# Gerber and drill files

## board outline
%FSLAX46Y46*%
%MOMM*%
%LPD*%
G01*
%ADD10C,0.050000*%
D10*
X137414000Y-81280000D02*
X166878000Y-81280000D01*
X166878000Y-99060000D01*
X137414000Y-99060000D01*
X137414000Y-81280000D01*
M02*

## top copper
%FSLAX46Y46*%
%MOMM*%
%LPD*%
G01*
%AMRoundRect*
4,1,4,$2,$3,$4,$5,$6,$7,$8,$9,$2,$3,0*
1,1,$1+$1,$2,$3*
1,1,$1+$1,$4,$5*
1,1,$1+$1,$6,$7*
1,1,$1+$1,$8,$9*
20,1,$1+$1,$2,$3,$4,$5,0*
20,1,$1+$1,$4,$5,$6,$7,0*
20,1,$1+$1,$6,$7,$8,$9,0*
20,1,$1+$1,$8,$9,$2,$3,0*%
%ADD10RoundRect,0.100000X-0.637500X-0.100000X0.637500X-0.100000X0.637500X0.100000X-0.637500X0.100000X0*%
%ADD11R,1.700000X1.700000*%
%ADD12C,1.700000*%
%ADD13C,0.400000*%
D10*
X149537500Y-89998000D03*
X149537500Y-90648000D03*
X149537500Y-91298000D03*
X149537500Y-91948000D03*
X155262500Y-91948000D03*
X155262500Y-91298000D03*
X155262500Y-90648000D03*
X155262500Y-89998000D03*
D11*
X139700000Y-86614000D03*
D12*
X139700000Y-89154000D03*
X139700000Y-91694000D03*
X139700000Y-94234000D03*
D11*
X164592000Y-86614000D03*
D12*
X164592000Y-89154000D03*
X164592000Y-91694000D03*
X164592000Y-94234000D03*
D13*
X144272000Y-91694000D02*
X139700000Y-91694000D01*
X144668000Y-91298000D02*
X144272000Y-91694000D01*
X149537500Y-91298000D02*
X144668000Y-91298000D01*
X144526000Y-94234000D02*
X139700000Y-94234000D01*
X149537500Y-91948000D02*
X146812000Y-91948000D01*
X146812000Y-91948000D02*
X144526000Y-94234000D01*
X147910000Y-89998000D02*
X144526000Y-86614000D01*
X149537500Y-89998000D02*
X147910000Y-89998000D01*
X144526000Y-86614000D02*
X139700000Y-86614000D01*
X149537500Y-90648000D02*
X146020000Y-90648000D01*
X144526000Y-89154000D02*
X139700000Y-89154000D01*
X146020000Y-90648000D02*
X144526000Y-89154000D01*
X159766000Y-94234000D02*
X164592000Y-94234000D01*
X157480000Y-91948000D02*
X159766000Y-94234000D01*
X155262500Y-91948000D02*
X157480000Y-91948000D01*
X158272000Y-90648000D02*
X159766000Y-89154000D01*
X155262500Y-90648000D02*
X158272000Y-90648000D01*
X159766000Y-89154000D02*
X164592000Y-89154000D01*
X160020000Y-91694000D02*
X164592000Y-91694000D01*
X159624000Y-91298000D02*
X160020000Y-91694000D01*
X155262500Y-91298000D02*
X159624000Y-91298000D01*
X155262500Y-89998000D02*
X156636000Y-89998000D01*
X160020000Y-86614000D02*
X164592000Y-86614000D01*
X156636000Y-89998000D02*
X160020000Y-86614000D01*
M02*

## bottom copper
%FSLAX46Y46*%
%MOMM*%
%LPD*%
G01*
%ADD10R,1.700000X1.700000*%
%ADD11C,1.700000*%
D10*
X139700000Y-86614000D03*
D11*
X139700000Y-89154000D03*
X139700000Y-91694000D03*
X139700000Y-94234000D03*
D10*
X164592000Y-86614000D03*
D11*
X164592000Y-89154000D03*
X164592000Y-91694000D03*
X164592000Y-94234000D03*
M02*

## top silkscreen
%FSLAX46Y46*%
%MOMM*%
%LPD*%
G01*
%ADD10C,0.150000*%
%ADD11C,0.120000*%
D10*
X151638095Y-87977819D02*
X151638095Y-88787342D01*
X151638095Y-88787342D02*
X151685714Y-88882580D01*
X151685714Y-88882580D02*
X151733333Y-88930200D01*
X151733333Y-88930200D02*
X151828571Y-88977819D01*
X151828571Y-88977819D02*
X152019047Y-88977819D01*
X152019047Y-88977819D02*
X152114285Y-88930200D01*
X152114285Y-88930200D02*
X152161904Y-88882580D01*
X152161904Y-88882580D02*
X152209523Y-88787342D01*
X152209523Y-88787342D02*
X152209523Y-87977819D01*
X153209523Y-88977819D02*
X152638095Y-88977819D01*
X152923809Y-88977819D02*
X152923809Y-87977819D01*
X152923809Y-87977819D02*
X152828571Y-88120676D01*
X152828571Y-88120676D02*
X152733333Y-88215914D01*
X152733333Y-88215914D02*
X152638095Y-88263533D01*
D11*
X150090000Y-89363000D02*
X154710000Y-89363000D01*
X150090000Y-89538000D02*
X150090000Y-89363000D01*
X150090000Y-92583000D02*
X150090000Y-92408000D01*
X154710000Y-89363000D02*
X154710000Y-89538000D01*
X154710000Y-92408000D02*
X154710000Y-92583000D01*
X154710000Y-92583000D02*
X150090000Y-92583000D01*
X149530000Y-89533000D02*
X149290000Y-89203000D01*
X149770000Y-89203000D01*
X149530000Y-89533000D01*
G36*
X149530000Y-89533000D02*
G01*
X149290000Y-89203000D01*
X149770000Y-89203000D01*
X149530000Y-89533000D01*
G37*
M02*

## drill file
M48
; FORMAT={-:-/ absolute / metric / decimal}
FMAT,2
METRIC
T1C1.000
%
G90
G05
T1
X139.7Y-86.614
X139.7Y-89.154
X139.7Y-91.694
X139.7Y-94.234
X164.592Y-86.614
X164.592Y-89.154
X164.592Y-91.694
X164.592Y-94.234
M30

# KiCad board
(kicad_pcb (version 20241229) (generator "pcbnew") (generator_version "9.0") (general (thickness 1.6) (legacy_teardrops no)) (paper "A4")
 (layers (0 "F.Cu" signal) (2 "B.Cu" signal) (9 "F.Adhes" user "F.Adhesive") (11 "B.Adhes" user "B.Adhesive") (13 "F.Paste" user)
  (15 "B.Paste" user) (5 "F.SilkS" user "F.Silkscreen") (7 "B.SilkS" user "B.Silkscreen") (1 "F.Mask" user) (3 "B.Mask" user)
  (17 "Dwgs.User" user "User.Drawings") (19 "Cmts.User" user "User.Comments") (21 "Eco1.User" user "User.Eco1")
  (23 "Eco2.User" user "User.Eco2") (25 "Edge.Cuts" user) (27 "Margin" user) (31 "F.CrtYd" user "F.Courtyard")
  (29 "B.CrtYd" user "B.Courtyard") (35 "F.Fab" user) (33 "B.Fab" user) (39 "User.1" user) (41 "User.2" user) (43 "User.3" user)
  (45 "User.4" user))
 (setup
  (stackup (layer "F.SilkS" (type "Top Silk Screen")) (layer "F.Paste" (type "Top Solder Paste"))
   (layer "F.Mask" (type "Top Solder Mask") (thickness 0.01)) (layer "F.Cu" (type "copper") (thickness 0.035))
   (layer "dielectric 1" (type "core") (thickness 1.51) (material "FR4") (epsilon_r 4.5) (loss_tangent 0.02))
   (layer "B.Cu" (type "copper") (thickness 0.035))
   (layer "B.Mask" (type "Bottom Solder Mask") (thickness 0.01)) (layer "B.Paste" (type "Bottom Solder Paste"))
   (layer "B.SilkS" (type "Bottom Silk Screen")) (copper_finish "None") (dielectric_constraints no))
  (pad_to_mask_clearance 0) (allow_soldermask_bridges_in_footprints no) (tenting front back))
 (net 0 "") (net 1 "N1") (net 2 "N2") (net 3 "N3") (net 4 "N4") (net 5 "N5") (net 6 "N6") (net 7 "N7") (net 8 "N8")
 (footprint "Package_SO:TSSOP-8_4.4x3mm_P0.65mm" (layer "F.Cu") (at 152.4 90.973)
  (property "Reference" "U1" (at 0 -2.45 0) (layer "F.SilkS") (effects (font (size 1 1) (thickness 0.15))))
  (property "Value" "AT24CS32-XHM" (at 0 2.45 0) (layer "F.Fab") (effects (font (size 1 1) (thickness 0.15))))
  (fp_line (start -2.31 -1.61) (end 2.31 -1.61) (stroke (width 0.12) (type solid)) (layer "F.SilkS"))
  (fp_line (start -2.31 -1.435) (end -2.31 -1.61) (stroke (width 0.12) (type solid)) (layer "F.SilkS"))
  (fp_line (start -2.31 1.61) (end -2.31 1.435) (stroke (width 0.12) (type solid)) (layer "F.SilkS"))
  (fp_line (start 2.31 -1.61) (end 2.31 -1.435) (stroke (width 0.12) (type solid)) (layer "F.SilkS"))
  (fp_line (start 2.31 1.435) (end 2.31 1.61) (stroke (width 0.12) (type solid)) (layer "F.SilkS"))
  (fp_line (start 2.31 1.61) (end -2.31 1.61) (stroke (width 0.12) (type solid)) (layer "F.SilkS"))
  (fp_poly (pts (xy -2.87 -1.44) (xy -3.11 -1.77) (xy -2.63 -1.77)) (stroke (width 0.12) (type solid)) (fill yes) (layer "F.SilkS"))
  (pad "1" smd roundrect (at -2.8625 -0.975) (size 1.475 0.4) (layers "F.Cu" "F.Mask" "F.Paste") (roundrect_rratio 0.25) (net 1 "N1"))
  (pad "2" smd roundrect (at -2.8625 -0.325) (size 1.475 0.4) (layers "F.Cu" "F.Mask" "F.Paste") (roundrect_rratio 0.25) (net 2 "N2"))
  (pad "3" smd roundrect (at -2.8625 0.325) (size 1.475 0.4) (layers "F.Cu" "F.Mask" "F.Paste") (roundrect_rratio 0.25) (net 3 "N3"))
  (pad "4" smd roundrect (at -2.8625 0.975) (size 1.475 0.4) (layers "F.Cu" "F.Mask" "F.Paste") (roundrect_rratio 0.25) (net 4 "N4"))
  (pad "5" smd roundrect (at 2.8625 0.975) (size 1.475 0.4) (layers "F.Cu" "F.Mask" "F.Paste") (roundrect_rratio 0.25) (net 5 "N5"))
  (pad "6" smd roundrect (at 2.8625 0.325) (size 1.475 0.4) (layers "F.Cu" "F.Mask" "F.Paste") (roundrect_rratio 0.25) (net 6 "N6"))
  (pad "7" smd roundrect (at 2.8625 -0.325) (size 1.475 0.4) (layers "F.Cu" "F.Mask" "F.Paste") (roundrect_rratio 0.25) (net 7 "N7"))
  (pad "8" smd roundrect (at 2.8625 -0.975) (size 1.475 0.4) (layers "F.Cu" "F.Mask" "F.Paste") (roundrect_rratio 0.25) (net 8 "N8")))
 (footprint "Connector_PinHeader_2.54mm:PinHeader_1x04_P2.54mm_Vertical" (layer "B.Cu") (at 139.7 86.614 180)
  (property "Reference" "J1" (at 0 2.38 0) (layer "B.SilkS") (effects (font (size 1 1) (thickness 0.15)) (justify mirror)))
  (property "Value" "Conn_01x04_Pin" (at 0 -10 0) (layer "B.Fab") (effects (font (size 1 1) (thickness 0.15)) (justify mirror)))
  (pad "1" thru_hole rect (at 0 0 180) (size 1.7 1.7) (drill 1) (layers "*.Cu" "*.Mask") (remove_unused_layers no) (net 1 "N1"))
  (pad "2" thru_hole circle (at 0 -2.54 180) (size 1.7 1.7) (drill 1) (layers "*.Cu" "*.Mask") (remove_unused_layers no) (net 2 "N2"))
  (pad "3" thru_hole circle (at 0 -5.08 180) (size 1.7 1.7) (drill 1) (layers "*.Cu" "*.Mask") (remove_unused_layers no) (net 3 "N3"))
  (pad "4" thru_hole circle (at 0 -7.62 180) (size 1.7 1.7) (drill 1) (layers "*.Cu" "*.Mask") (remove_unused_layers no) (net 4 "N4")))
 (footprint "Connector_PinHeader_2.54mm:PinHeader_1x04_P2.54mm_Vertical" (layer "B.Cu") (at 164.592 86.614 180)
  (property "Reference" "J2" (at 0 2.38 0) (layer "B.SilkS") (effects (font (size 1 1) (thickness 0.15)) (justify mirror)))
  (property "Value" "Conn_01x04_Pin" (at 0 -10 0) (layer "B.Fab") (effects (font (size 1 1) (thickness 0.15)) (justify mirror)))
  (pad "1" thru_hole rect (at 0 0 180) (size 1.7 1.7) (drill 1) (layers "*.Cu" "*.Mask") (remove_unused_layers no) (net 8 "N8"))
  (pad "2" thru_hole circle (at 0 -2.54 180) (size 1.7 1.7) (drill 1) (layers "*.Cu" "*.Mask") (remove_unused_layers no) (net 7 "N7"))
  (pad "3" thru_hole circle (at 0 -5.08 180) (size 1.7 1.7) (drill 1) (layers "*.Cu" "*.Mask") (remove_unused_layers no) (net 6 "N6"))
  (pad "4" thru_hole circle (at 0 -7.62 180) (size 1.7 1.7) (drill 1) (layers "*.Cu" "*.Mask") (remove_unused_layers no) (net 5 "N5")))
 (gr_rect (start 137.414 81.28) (end 166.878 99.06) (stroke (width 0.05) (type default)) (fill no) (layer "Edge.Cuts"))
 (segment (start 144.272 91.694) (end 139.7 91.694) (width 0.4) (layer "F.Cu") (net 3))
 (segment (start 144.668 91.298) (end 144.272 91.694) (width 0.4) (layer "F.Cu") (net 3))
 (segment (start 149.5375 91.298) (end 144.668 91.298) (width 0.4) (layer "F.Cu") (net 3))
 (segment (start 144.526 94.234) (end 139.7 94.234) (width 0.4) (layer "F.Cu") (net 4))
 (segment (start 149.5375 91.948) (end 146.812 91.948) (width 0.4) (layer "F.Cu") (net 4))
 (segment (start 146.812 91.948) (end 144.526 94.234) (width 0.4) (layer "F.Cu") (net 4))
 (segment (start 147.91 89.998) (end 144.526 86.614) (width 0.4) (layer "F.Cu") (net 1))
 (segment (start 149.5375 89.998) (end 147.91 89.998) (width 0.4) (layer "F.Cu") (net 1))
 (segment (start 144.526 86.614) (end 139.7 86.614) (width 0.4) (layer "F.Cu") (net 1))
 (segment (start 149.5375 90.648) (end 146.02 90.648) (width 0.4) (layer "F.Cu") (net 2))
 (segment (start 144.526 89.154) (end 139.7 89.154) (width 0.4) (layer "F.Cu") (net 2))
 (segment (start 146.02 90.648) (end 144.526 89.154) (width 0.4) (layer "F.Cu") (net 2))
 (segment (start 159.766 94.234) (end 164.592 94.234) (width 0.4) (layer "F.Cu") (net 5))
 (segment (start 157.48 91.948) (end 159.766 94.234) (width 0.4) (layer "F.Cu") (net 5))
 (segment (start 155.2625 91.948) (end 157.48 91.948) (width 0.4) (layer "F.Cu") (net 5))
 (segment (start 158.272 90.648) (end 159.766 89.154) (width 0.4) (layer "F.Cu") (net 7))
 (segment (start 155.2625 90.648) (end 158.272 90.648) (width 0.4) (layer "F.Cu") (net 7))
 (segment (start 159.766 89.154) (end 164.592 89.154) (width 0.4) (layer "F.Cu") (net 7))
 (segment (start 160.02 91.694) (end 164.592 91.694) (width 0.4) (layer "F.Cu") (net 6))
 (segment (start 159.624 91.298) (end 160.02 91.694) (width 0.4) (layer "F.Cu") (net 6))
 (segment (start 155.2625 91.298) (end 159.624 91.298) (width 0.4) (layer "F.Cu") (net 6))
 (segment (start 155.2625 89.998) (end 156.636 89.998) (width 0.4) (layer "F.Cu") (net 8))
 (segment (start 160.02 86.614) (end 164.592 86.614) (width 0.4) (layer "F.Cu") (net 8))
 (segment (start 156.636 89.998) (end 160.02 86.614) (width 0.4) (layer "F.Cu") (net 8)))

